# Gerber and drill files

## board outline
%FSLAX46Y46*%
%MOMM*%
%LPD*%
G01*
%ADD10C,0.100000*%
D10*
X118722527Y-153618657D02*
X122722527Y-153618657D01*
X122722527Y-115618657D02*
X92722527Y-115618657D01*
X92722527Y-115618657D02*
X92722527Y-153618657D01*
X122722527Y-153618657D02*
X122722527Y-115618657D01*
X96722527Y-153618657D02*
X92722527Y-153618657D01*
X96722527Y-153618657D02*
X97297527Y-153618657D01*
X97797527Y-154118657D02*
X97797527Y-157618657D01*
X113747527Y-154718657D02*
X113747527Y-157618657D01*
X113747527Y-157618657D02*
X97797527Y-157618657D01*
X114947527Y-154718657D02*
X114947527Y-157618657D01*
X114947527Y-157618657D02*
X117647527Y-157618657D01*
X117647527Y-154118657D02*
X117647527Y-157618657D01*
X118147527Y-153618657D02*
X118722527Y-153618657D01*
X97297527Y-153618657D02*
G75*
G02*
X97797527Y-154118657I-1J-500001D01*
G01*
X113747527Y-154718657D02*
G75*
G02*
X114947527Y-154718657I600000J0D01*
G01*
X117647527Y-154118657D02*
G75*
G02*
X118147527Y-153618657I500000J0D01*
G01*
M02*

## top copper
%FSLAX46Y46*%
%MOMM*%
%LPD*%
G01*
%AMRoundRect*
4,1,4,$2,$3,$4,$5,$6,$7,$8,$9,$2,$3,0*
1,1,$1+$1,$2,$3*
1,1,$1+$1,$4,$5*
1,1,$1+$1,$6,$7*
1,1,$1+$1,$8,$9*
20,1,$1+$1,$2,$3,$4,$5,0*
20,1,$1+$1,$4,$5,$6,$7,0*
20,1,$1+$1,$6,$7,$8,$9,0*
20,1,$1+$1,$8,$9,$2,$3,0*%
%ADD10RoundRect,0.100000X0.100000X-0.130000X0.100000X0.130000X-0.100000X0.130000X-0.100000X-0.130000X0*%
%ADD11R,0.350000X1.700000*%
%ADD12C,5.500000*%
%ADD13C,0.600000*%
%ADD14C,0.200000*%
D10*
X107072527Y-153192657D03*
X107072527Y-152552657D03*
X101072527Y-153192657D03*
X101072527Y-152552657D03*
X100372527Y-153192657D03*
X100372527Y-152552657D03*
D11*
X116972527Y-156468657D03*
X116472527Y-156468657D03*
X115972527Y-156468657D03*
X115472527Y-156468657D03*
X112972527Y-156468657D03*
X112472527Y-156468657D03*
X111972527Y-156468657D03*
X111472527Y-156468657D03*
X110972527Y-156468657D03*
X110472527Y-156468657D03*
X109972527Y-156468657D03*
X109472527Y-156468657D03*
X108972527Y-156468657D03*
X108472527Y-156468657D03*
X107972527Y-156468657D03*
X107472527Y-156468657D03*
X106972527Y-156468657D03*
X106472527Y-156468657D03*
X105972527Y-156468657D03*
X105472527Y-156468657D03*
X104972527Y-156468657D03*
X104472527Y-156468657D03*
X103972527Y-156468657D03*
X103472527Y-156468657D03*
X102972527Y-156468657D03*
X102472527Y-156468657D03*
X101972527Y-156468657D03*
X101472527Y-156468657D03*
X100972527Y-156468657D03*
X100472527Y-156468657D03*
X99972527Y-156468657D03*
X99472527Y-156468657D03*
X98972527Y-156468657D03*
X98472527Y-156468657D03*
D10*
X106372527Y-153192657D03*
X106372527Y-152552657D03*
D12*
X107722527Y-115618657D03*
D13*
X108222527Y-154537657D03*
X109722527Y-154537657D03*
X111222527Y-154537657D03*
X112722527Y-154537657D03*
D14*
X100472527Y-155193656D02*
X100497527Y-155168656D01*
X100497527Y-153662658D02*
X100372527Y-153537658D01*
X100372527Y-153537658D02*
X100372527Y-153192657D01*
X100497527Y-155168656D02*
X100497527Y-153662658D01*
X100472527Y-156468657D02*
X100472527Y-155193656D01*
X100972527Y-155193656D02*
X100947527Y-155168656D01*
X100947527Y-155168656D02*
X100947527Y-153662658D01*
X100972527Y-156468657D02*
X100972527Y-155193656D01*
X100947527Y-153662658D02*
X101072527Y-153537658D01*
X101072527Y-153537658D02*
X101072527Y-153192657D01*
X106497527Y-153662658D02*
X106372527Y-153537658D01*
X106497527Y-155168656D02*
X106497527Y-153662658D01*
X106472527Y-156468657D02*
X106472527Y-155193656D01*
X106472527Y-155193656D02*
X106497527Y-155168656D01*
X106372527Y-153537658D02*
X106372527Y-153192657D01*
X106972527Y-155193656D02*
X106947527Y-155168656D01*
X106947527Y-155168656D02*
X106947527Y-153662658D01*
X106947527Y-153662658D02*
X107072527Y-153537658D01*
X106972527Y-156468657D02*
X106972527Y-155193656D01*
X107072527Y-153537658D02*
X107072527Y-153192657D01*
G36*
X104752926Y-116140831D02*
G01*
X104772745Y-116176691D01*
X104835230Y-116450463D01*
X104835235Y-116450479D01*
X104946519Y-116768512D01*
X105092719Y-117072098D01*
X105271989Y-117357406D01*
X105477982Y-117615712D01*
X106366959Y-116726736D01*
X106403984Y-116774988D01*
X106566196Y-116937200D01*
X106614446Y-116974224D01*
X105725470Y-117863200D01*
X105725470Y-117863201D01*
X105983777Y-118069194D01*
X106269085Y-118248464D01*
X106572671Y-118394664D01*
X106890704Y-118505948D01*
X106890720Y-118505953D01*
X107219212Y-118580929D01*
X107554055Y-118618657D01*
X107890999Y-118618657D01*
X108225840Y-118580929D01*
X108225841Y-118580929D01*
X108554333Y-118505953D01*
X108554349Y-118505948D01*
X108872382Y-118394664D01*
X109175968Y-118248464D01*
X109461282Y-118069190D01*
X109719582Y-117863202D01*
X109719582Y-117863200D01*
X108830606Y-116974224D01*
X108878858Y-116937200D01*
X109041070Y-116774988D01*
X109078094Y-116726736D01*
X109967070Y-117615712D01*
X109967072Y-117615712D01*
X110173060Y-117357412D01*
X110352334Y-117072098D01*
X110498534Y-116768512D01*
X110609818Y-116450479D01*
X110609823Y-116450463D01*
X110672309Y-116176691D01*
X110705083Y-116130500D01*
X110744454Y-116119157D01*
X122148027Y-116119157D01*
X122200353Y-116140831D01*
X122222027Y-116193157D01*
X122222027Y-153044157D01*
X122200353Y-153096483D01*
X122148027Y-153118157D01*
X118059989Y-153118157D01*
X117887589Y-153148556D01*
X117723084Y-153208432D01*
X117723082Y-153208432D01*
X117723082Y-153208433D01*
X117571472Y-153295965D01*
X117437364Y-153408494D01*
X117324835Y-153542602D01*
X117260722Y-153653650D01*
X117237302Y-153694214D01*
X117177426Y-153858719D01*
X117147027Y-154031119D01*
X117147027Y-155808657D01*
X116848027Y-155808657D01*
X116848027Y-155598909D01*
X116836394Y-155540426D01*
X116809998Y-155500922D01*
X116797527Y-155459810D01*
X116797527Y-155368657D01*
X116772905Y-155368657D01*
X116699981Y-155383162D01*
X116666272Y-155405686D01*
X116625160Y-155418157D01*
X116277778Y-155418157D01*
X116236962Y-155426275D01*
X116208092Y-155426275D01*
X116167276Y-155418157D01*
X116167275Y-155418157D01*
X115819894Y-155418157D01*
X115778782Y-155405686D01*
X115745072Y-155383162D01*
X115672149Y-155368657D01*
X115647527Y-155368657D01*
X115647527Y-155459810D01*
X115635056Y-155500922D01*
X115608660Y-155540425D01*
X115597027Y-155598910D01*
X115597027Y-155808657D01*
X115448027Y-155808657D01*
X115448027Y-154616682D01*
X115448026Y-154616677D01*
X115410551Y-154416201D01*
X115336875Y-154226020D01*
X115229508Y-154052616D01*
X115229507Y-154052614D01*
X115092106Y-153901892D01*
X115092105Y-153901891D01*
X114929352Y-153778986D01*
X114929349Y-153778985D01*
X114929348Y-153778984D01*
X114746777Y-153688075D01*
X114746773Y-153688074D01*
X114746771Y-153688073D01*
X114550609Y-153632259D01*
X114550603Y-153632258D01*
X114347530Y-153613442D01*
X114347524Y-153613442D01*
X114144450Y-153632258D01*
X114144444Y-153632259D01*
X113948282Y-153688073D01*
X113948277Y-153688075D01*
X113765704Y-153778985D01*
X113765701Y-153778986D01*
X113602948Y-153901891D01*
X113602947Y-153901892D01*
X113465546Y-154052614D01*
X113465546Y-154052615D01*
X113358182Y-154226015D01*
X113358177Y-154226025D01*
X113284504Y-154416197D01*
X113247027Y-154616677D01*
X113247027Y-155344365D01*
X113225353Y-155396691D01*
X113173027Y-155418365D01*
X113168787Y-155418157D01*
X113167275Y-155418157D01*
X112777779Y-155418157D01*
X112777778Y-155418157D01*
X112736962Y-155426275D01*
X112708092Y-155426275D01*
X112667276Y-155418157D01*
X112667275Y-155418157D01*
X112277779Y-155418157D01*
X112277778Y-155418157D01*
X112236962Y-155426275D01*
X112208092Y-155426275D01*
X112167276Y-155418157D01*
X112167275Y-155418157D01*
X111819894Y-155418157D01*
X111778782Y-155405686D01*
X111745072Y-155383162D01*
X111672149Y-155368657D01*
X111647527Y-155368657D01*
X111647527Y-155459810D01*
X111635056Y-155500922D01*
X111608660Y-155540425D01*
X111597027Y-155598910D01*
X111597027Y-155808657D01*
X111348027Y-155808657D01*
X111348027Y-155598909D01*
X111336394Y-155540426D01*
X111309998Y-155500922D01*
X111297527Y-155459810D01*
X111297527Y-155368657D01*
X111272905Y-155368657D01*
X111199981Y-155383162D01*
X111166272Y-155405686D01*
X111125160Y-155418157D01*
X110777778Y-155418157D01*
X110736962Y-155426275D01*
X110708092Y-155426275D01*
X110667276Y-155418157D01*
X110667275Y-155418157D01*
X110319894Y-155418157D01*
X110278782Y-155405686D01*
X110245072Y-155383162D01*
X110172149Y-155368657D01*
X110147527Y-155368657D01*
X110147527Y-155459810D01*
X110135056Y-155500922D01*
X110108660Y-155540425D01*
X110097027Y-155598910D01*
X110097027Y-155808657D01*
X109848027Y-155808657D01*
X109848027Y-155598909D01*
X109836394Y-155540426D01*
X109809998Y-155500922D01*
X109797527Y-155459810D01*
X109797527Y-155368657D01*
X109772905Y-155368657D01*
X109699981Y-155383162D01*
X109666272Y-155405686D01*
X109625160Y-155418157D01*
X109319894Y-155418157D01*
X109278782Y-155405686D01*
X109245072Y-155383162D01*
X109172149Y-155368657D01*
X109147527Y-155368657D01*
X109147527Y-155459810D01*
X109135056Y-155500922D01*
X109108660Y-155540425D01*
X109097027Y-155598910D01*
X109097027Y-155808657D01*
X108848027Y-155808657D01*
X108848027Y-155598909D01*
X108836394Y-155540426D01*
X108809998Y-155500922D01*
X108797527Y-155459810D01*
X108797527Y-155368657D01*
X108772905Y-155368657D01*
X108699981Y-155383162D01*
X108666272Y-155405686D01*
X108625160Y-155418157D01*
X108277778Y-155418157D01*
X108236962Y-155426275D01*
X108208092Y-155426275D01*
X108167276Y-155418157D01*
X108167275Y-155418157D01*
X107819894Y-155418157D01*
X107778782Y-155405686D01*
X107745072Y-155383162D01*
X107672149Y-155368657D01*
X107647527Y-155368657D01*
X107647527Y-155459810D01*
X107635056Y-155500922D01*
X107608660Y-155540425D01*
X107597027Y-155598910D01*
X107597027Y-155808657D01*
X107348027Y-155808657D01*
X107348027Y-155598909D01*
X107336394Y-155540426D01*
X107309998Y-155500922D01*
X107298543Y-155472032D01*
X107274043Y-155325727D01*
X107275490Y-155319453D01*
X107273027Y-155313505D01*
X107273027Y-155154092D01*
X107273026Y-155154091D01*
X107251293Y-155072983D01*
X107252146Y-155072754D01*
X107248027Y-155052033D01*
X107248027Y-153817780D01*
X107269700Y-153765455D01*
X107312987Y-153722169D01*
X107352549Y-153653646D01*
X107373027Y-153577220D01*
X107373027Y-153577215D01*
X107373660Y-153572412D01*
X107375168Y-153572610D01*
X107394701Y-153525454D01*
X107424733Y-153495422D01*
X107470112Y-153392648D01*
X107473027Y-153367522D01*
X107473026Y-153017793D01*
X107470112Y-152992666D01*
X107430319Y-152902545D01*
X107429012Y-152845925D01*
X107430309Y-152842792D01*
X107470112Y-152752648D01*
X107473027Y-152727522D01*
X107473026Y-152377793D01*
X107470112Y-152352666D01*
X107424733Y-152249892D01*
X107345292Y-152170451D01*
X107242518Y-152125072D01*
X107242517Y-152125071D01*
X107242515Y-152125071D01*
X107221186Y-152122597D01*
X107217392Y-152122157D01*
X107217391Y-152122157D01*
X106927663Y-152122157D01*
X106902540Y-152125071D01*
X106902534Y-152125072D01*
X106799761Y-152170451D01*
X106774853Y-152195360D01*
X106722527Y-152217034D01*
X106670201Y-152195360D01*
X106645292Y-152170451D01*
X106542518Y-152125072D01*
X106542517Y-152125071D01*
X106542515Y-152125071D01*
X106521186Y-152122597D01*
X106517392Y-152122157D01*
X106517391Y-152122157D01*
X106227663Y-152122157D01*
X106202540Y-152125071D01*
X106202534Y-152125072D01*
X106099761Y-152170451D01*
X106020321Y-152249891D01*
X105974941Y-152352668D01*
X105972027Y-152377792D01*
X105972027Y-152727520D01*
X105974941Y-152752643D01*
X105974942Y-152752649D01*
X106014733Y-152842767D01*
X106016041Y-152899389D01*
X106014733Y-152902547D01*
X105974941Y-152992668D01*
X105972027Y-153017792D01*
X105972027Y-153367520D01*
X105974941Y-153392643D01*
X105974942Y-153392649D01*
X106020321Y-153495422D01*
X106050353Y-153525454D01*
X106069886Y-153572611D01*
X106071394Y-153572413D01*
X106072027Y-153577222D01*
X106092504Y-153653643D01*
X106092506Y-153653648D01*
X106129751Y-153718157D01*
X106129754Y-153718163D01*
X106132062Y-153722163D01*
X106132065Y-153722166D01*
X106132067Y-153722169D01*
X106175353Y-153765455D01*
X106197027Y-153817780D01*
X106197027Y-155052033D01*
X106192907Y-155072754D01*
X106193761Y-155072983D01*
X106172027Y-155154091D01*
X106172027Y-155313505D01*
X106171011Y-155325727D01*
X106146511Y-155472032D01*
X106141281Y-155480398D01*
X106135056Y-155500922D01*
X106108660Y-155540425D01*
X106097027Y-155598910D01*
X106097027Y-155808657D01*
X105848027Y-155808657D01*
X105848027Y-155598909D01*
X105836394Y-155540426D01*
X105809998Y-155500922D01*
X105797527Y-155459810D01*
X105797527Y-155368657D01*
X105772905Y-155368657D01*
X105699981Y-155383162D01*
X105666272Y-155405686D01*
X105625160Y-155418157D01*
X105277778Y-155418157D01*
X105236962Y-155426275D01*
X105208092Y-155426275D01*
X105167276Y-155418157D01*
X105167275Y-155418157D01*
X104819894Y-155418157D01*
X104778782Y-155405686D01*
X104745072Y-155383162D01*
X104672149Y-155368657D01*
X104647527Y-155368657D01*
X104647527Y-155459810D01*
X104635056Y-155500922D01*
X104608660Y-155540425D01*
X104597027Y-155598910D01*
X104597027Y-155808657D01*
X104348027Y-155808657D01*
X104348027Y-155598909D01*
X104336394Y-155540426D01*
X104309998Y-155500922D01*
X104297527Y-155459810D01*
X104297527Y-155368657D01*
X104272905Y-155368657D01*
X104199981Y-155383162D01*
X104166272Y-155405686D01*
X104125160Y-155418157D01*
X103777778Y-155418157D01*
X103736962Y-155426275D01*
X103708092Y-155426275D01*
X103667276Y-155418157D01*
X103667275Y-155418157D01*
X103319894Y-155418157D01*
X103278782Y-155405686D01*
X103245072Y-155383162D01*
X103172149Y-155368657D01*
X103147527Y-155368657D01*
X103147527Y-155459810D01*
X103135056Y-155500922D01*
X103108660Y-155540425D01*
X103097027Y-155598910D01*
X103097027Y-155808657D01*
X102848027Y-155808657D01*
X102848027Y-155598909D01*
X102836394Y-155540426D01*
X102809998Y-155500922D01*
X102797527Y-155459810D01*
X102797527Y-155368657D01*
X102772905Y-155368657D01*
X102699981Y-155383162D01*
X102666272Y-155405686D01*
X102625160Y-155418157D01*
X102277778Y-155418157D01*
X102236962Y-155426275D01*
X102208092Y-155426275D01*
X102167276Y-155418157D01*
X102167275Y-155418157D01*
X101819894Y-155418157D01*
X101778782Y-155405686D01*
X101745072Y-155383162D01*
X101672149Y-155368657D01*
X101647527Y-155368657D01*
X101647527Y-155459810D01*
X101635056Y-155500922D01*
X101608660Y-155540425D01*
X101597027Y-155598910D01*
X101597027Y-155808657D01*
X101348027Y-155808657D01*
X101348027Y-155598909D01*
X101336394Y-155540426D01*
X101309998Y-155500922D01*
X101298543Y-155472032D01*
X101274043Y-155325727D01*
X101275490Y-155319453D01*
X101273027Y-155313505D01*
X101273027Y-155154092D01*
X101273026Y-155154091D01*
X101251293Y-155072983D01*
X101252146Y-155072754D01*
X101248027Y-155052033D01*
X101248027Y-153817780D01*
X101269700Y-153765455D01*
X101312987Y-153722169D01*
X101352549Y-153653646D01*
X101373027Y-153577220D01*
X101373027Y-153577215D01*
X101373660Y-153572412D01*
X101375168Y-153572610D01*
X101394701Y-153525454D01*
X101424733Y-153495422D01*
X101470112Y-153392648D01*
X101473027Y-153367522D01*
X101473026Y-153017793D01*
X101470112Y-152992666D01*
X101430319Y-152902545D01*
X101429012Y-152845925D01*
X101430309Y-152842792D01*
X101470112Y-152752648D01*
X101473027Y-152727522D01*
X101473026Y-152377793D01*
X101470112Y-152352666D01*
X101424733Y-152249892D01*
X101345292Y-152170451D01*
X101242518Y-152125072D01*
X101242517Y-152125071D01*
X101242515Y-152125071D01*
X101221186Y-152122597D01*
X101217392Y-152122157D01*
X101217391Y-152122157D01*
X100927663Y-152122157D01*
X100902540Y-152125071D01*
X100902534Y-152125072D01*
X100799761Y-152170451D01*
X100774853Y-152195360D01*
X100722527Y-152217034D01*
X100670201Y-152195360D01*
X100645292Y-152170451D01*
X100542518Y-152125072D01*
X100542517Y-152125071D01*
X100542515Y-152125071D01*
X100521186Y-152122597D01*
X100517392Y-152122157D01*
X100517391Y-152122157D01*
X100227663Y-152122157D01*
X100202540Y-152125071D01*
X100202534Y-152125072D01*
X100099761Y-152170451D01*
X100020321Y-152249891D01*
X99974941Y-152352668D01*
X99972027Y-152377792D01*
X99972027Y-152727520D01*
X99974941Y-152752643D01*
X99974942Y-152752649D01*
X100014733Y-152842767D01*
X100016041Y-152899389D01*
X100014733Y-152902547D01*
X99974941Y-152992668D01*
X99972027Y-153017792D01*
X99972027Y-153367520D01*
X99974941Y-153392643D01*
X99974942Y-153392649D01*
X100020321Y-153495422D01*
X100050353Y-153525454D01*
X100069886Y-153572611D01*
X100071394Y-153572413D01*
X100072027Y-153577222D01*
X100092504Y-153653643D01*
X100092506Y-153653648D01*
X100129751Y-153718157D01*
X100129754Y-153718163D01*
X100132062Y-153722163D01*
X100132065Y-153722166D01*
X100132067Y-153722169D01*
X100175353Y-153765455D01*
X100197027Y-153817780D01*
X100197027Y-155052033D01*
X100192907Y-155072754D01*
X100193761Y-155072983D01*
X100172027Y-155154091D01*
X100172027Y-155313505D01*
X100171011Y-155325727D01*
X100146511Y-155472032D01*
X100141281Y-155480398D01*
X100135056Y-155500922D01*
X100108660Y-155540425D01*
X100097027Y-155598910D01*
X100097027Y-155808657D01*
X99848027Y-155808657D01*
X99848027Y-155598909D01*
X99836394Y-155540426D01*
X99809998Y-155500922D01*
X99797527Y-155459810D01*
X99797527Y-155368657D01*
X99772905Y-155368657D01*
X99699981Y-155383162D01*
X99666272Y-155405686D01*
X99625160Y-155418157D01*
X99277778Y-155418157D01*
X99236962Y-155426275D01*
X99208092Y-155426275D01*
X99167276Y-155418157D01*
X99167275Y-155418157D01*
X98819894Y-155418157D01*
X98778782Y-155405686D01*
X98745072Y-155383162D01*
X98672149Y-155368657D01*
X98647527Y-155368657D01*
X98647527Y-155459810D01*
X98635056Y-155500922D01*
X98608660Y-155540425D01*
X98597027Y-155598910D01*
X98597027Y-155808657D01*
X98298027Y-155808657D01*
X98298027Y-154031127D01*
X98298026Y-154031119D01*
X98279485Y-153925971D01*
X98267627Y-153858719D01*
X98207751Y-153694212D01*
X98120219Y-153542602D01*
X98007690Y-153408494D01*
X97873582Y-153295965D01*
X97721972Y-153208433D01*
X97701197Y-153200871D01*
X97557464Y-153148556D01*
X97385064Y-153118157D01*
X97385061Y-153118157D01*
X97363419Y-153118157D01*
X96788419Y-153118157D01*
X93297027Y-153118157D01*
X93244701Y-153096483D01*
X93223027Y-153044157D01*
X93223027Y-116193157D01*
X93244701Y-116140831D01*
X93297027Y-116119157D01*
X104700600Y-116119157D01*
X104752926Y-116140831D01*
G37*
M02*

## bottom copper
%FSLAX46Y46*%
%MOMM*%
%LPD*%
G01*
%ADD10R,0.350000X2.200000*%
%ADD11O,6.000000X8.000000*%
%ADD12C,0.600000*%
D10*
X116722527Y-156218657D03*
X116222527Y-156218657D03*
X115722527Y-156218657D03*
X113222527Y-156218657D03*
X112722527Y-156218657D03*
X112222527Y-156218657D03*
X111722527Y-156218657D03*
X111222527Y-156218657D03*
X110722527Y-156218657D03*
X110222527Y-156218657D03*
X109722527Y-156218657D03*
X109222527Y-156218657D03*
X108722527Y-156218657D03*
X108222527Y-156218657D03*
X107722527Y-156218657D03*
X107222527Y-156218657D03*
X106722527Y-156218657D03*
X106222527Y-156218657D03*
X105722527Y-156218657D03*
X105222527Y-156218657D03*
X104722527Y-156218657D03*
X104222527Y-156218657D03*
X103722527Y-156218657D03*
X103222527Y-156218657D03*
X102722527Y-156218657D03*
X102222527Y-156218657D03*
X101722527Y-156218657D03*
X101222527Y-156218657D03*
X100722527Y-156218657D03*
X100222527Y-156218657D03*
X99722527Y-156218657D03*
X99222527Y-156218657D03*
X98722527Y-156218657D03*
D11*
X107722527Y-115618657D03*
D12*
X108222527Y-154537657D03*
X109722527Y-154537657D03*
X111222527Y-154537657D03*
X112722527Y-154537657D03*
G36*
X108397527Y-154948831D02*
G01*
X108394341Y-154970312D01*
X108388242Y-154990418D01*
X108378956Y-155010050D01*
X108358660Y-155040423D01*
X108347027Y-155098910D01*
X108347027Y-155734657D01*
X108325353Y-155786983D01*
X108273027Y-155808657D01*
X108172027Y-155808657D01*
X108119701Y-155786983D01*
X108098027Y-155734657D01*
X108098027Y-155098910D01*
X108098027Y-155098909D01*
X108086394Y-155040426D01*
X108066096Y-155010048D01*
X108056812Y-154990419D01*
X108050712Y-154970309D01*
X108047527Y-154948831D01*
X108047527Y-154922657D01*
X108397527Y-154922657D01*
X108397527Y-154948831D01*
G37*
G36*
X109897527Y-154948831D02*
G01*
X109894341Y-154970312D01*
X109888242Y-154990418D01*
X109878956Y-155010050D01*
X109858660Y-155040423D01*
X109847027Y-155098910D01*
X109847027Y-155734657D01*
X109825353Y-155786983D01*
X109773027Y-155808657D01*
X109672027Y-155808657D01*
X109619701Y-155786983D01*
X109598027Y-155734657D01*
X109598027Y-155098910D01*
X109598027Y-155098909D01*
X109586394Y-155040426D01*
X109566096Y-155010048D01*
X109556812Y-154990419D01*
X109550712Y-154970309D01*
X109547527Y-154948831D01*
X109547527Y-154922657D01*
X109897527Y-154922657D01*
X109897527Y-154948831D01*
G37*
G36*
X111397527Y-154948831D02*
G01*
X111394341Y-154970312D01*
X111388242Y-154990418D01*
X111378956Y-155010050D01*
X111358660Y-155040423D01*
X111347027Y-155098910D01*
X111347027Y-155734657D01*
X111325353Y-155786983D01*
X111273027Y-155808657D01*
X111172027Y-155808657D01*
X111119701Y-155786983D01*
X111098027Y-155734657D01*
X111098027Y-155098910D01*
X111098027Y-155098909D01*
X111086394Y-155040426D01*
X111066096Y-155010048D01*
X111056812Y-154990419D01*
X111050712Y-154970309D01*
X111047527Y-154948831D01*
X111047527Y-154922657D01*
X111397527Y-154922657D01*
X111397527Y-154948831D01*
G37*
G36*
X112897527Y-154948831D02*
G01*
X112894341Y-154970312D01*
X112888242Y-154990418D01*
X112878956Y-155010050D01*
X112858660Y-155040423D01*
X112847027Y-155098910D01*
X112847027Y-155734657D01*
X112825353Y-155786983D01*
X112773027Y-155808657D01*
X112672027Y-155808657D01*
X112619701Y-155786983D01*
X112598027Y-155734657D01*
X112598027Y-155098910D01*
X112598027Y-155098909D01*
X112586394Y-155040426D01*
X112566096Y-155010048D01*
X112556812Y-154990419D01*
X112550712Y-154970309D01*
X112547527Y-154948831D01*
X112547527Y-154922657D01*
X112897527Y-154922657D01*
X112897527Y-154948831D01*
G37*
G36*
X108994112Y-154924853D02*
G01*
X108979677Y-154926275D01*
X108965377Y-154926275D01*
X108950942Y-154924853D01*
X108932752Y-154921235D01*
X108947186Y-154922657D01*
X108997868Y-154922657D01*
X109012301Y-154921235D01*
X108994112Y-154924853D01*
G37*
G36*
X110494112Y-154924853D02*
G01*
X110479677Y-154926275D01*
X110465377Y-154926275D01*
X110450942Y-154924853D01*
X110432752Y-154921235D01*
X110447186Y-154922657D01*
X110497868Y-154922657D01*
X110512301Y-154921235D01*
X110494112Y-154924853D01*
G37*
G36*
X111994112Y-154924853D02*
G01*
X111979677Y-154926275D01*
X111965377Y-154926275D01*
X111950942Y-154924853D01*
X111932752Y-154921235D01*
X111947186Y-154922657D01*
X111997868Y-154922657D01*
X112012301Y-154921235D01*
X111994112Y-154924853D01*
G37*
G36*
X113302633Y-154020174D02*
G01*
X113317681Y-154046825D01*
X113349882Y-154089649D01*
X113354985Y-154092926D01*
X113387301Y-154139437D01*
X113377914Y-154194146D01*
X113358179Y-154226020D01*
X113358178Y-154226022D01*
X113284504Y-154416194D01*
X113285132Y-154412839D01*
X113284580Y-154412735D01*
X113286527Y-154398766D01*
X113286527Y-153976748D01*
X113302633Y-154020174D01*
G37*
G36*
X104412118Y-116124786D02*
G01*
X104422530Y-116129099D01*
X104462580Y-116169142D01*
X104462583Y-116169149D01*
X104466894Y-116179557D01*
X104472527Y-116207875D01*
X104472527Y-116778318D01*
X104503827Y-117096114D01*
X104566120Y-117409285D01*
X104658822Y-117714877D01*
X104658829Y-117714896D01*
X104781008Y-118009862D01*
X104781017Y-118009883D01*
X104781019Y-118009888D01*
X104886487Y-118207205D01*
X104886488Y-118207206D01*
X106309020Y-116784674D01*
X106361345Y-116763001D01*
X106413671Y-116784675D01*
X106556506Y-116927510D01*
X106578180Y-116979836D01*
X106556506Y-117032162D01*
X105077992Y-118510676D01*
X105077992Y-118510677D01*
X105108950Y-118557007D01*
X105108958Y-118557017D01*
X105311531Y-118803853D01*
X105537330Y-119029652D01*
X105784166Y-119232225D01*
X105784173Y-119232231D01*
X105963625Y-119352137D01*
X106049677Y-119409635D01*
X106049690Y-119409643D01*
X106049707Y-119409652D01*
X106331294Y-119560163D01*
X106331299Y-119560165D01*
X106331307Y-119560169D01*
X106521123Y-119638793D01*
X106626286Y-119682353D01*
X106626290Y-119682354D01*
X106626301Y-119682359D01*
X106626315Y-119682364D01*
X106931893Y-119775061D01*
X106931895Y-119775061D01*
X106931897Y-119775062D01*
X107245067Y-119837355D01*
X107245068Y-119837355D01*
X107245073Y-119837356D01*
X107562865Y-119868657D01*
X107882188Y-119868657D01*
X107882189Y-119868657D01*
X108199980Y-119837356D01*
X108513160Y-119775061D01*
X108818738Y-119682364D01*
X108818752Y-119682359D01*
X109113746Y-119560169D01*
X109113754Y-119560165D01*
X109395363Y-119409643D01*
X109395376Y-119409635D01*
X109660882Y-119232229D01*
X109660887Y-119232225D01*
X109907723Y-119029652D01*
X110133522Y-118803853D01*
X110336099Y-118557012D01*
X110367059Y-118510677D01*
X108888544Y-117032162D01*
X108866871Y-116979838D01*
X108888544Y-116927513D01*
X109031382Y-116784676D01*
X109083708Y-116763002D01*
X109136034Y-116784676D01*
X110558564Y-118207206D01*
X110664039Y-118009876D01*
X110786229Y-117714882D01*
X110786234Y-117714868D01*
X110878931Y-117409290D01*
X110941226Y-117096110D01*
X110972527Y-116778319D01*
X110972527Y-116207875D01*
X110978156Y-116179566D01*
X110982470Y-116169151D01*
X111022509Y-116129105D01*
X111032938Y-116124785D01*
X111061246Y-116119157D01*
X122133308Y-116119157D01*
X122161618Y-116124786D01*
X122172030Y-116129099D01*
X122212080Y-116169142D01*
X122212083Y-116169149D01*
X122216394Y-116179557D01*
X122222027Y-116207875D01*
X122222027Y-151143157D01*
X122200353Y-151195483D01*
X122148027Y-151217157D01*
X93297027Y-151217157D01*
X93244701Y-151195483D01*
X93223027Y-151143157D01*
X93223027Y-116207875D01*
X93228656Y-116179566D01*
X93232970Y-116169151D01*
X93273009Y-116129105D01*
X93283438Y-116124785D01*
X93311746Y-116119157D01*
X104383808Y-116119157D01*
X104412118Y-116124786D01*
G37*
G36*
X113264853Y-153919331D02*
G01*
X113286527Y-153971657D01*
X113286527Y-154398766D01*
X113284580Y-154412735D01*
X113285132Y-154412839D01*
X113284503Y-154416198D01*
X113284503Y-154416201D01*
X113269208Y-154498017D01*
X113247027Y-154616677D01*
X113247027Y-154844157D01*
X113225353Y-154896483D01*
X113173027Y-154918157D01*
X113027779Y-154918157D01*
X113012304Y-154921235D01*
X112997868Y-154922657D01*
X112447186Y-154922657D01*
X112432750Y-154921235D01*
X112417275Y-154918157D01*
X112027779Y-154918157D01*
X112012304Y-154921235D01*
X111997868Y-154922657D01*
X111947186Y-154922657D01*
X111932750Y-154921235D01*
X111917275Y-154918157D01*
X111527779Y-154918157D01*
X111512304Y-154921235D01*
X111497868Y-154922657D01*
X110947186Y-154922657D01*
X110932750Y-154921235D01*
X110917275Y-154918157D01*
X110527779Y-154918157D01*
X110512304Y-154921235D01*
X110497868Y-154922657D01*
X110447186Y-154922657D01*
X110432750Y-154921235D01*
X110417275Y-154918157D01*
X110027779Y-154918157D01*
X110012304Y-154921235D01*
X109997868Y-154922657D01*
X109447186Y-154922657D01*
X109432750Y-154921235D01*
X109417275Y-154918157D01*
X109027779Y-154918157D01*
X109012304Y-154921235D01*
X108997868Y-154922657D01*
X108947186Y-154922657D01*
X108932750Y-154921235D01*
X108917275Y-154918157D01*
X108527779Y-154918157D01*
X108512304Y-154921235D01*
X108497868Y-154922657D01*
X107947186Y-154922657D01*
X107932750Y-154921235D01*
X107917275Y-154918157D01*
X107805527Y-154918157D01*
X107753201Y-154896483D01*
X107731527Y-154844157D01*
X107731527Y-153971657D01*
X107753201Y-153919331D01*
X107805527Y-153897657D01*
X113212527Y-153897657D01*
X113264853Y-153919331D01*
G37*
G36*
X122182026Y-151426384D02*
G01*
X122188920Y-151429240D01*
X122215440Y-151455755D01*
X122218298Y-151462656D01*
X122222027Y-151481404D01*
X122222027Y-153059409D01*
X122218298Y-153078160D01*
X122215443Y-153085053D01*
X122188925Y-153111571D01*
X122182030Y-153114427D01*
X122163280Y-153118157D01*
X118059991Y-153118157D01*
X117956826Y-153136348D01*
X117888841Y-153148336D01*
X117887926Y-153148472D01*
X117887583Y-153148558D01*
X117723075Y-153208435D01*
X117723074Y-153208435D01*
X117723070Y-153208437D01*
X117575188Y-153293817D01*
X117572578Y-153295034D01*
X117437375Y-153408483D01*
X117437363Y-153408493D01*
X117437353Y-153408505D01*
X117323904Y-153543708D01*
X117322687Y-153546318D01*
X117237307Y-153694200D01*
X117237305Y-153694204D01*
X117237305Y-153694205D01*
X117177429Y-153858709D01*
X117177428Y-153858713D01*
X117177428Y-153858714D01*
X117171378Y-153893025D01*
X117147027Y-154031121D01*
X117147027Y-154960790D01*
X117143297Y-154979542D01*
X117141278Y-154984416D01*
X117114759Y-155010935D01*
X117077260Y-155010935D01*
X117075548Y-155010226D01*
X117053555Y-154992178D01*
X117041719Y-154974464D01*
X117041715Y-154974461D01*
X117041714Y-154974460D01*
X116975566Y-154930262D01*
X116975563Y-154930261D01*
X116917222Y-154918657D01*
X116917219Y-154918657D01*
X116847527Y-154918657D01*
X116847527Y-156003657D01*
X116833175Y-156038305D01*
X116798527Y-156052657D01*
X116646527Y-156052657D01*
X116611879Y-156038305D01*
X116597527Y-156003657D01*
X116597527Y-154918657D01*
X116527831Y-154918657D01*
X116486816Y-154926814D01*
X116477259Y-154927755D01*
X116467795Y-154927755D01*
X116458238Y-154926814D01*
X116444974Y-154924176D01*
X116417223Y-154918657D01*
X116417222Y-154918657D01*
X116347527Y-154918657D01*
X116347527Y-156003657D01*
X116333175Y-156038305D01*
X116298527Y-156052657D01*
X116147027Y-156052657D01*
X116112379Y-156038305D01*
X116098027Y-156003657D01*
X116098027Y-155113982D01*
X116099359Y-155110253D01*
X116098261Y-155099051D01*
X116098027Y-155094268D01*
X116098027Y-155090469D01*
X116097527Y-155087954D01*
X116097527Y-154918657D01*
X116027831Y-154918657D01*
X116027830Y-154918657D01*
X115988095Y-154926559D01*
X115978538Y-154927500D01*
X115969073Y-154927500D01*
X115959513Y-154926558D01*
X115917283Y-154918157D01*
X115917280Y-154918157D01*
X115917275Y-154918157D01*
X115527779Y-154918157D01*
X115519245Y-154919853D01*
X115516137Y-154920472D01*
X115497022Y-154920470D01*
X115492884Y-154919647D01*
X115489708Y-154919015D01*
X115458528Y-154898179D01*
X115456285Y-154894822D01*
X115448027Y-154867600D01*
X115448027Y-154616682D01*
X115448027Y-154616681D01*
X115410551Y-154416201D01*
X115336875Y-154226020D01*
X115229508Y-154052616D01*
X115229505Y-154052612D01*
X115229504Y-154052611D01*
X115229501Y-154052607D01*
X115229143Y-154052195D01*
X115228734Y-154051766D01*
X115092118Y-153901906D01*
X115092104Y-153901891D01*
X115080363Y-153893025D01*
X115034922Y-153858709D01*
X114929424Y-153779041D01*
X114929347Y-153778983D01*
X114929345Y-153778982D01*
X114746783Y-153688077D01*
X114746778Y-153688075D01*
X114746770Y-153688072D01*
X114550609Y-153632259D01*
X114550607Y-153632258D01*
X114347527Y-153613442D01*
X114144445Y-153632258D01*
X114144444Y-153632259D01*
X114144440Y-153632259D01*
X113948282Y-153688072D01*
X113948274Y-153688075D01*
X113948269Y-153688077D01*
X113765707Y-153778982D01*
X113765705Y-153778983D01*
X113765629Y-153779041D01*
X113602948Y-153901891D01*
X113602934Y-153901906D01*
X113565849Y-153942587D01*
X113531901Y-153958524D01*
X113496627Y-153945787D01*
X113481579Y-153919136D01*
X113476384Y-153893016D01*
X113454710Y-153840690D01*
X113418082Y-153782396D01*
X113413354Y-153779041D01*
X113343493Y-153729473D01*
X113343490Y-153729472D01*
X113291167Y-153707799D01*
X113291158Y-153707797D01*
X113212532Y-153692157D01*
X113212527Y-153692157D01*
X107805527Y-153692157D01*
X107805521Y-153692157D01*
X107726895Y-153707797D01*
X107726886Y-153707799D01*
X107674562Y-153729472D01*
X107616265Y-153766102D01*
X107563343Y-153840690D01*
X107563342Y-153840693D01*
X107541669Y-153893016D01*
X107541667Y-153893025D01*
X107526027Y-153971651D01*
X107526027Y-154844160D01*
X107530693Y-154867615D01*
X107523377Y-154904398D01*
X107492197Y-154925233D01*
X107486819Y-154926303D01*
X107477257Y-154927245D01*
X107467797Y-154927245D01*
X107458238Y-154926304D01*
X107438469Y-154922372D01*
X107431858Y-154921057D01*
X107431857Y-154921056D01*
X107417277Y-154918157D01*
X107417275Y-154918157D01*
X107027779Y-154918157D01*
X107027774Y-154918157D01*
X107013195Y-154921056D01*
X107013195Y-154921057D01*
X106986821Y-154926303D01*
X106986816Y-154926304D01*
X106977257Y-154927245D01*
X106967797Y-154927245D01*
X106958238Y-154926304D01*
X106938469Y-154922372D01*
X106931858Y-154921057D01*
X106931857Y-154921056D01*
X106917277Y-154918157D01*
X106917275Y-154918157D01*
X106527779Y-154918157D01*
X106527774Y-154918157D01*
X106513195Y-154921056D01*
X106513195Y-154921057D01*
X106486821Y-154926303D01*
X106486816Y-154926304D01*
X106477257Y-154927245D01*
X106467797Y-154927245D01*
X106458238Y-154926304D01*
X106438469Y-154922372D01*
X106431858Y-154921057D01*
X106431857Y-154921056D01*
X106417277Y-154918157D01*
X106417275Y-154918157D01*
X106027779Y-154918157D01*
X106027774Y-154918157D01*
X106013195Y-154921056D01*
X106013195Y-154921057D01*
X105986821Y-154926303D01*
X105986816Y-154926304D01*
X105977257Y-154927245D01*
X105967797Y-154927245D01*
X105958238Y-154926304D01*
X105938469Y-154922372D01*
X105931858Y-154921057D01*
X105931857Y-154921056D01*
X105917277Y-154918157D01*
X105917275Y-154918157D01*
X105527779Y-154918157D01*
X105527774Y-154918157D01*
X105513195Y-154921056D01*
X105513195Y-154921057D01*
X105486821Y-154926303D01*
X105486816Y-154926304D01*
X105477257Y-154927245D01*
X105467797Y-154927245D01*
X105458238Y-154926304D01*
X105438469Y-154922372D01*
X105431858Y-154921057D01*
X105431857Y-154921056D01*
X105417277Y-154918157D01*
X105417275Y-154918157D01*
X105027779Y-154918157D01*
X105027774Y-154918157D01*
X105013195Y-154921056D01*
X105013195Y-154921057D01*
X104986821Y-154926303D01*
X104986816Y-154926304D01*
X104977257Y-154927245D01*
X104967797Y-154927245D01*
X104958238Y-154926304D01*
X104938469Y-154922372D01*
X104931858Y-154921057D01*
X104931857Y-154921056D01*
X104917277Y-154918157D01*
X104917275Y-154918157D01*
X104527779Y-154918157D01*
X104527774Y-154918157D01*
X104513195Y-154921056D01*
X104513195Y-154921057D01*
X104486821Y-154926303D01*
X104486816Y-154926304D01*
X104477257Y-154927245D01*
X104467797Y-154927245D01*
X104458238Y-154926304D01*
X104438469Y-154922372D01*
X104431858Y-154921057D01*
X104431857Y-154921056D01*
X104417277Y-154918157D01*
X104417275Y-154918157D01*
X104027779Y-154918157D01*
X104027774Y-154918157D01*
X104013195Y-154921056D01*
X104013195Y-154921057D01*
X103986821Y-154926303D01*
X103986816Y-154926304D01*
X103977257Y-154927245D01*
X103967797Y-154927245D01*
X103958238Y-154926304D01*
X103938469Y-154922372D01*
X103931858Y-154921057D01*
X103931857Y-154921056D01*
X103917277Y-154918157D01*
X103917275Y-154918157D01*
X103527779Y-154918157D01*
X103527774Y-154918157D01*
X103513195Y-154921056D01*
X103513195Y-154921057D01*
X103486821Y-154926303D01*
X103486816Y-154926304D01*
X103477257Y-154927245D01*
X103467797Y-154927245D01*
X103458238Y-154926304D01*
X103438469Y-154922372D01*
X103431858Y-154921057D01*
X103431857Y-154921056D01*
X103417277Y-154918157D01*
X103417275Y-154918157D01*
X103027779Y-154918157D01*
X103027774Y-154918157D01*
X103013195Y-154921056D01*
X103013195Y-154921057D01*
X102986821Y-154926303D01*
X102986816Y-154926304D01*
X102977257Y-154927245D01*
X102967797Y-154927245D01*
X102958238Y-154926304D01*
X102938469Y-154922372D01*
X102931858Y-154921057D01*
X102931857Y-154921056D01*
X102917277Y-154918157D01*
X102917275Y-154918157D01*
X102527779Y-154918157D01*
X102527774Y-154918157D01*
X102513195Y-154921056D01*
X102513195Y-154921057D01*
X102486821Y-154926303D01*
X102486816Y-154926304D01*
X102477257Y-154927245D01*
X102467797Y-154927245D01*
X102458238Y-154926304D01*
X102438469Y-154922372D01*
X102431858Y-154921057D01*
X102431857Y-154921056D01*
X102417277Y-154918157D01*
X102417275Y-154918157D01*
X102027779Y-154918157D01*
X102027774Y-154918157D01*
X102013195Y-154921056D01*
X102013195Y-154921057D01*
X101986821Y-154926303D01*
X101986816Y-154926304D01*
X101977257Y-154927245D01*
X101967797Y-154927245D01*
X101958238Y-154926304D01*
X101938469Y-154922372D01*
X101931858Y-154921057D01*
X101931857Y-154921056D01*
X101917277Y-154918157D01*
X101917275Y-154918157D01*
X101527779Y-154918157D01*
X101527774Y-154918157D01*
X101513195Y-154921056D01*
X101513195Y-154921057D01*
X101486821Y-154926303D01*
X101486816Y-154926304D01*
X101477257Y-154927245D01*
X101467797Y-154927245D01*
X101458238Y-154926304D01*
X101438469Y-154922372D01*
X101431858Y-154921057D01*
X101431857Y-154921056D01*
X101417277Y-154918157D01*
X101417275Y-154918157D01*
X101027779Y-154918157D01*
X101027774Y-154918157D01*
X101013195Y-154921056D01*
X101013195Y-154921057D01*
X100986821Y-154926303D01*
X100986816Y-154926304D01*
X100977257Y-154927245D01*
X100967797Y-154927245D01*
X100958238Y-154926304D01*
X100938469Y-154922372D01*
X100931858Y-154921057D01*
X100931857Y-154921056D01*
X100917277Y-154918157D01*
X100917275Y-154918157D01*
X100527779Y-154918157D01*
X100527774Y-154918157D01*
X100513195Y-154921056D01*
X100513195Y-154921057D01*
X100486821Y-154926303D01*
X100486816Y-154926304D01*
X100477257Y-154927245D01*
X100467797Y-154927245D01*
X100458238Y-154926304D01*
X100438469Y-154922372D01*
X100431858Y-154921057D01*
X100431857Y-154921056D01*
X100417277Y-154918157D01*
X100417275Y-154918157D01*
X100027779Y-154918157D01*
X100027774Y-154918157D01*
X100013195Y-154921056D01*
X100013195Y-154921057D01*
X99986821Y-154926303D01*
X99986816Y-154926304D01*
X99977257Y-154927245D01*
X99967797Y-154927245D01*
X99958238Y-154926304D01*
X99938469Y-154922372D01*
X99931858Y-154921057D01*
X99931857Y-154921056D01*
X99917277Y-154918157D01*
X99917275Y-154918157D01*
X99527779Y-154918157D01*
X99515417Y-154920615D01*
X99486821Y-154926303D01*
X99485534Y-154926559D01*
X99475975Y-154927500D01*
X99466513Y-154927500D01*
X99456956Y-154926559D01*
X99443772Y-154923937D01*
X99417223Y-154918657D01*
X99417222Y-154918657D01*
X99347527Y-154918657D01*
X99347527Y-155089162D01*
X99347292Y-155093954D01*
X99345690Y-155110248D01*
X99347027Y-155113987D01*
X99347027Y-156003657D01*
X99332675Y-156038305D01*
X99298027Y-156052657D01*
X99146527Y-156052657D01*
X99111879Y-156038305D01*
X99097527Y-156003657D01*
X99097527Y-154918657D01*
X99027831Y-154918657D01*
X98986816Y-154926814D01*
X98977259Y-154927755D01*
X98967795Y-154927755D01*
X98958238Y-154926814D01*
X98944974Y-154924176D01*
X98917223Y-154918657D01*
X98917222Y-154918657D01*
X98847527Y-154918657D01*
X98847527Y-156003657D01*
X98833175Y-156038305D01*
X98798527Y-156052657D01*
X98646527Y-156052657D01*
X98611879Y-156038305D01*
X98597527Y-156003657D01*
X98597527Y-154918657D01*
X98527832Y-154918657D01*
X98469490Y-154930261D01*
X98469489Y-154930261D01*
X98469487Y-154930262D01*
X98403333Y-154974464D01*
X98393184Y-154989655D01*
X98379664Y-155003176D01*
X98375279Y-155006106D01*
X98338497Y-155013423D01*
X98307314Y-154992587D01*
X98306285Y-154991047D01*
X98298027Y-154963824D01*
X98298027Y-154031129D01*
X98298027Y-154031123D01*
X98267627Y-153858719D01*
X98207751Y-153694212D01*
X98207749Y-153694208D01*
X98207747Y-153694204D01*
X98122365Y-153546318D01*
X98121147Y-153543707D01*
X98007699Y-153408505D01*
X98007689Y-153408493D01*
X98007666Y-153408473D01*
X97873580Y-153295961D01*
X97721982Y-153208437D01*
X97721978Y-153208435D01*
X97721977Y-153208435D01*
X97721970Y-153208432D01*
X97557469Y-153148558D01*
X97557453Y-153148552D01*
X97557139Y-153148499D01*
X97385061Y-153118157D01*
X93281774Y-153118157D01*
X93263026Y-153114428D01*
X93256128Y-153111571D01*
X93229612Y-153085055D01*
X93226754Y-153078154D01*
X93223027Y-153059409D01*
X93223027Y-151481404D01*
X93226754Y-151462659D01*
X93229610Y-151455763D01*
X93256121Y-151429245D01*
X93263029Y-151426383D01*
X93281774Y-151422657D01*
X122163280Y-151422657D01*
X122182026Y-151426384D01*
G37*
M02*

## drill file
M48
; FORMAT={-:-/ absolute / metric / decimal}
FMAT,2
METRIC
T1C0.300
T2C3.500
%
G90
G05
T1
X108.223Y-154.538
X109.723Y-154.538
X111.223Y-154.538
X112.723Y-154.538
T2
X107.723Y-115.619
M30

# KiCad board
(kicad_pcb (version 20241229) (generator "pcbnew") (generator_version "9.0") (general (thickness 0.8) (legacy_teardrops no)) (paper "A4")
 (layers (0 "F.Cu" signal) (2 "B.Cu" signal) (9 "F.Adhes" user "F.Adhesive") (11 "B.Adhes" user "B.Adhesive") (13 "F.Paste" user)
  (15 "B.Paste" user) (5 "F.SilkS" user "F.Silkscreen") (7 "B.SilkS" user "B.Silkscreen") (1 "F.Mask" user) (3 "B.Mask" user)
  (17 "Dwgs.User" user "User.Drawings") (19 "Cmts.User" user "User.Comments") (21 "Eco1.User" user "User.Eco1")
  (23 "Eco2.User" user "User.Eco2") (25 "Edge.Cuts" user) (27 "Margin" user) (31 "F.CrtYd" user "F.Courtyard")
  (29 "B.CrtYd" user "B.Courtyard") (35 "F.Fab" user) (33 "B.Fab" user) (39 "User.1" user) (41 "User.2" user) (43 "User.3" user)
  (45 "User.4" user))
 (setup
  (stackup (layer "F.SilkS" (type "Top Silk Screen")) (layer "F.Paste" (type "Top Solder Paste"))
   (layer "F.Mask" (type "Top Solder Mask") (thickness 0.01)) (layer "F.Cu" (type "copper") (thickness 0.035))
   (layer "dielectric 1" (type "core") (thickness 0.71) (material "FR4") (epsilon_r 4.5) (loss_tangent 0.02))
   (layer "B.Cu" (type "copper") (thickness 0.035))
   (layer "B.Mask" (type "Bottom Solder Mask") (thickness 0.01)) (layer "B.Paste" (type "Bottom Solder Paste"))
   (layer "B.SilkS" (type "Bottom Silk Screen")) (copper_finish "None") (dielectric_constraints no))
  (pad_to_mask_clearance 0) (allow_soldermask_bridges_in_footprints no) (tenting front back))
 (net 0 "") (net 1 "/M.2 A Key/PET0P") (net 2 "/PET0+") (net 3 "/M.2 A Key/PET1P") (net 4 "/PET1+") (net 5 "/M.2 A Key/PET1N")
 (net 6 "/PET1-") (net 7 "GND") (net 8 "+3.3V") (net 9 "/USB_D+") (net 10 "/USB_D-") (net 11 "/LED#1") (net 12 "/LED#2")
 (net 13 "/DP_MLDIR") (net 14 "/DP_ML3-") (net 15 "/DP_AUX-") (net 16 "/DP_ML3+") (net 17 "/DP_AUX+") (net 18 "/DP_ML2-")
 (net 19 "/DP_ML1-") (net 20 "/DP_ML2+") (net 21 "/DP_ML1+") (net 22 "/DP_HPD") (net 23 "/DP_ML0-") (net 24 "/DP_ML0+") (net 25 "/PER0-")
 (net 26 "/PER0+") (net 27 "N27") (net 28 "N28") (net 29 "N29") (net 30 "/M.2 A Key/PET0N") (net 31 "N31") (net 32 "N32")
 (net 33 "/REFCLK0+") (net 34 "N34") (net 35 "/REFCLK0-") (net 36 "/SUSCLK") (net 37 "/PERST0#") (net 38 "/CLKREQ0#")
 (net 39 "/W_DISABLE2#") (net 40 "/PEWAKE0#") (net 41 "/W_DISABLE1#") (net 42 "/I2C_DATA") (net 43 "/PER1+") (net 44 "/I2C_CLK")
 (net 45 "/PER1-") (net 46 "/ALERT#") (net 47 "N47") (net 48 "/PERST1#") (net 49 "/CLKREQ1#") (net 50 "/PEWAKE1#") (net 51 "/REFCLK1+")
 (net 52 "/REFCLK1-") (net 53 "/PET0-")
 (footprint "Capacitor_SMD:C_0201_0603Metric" (layer "F.Cu") (at 107.072527 152.872657 90)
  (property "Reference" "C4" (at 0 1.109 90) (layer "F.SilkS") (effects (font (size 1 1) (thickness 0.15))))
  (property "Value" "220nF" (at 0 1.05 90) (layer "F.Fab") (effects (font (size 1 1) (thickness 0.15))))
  (pad "" smd roundrect (at -0.345 0 90) (size 0.318 0.36) (layers "F.Paste") (roundrect_rratio 0.25))
  (pad "" smd roundrect (at 0.345 0 90) (size 0.318 0.36) (layers "F.Paste") (roundrect_rratio 0.25))
  (pad "1" smd roundrect (at -0.32 0 90) (size 0.46 0.4) (layers "F.Cu" "F.Mask") (roundrect_rratio 0.25) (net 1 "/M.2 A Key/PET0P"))
  (pad "2" smd roundrect (at 0.32 0 90) (size 0.46 0.4) (layers "F.Cu" "F.Mask") (roundrect_rratio 0.25) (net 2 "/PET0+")))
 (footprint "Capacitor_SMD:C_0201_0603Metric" (layer "F.Cu") (at 101.072527 152.872657 90)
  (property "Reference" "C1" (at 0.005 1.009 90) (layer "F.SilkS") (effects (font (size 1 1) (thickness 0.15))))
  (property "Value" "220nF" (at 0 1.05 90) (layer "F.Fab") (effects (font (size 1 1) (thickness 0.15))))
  (pad "" smd roundrect (at -0.345 0 90) (size 0.318 0.36) (layers "F.Paste") (roundrect_rratio 0.25))
  (pad "" smd roundrect (at 0.345 0 90) (size 0.318 0.36) (layers "F.Paste") (roundrect_rratio 0.25))
  (pad "1" smd roundrect (at -0.32 0 90) (size 0.46 0.4) (layers "F.Cu" "F.Mask") (roundrect_rratio 0.25) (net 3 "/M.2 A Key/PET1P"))
  (pad "2" smd roundrect (at 0.32 0 90) (size 0.46 0.4) (layers "F.Cu" "F.Mask") (roundrect_rratio 0.25) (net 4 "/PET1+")))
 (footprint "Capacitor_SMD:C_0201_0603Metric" (layer "F.Cu") (at 100.372527 152.872657 90)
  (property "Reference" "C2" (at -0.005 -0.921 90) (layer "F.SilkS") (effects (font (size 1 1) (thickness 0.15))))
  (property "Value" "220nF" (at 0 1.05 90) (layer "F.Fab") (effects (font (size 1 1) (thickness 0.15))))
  (pad "" smd roundrect (at -0.345 0 90) (size 0.318 0.36) (layers "F.Paste") (roundrect_rratio 0.25))
  (pad "" smd roundrect (at 0.345 0 90) (size 0.318 0.36) (layers "F.Paste") (roundrect_rratio 0.25))
  (pad "1" smd roundrect (at -0.32 0 90) (size 0.46 0.4) (layers "F.Cu" "F.Mask") (roundrect_rratio 0.25) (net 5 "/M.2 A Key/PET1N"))
  (pad "2" smd roundrect (at 0.32 0 90) (size 0.46 0.4) (layers "F.Cu" "F.Mask") (roundrect_rratio 0.25) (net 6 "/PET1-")))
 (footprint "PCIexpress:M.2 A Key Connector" (layer "F.Cu") (at 107.722527 156.508657)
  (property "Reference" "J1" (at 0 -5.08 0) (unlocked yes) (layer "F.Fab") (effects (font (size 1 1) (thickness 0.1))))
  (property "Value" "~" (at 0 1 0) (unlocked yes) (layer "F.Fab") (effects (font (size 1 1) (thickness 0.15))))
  (fp_line (start -11 -2.89) (end -10.425 -2.89) (stroke (width 0.1) (type default)) (layer "Edge.Cuts"))
  (fp_line (start -9.925 -2.39) (end -9.925 1.11) (stroke (width 0.1) (type default)) (layer "Edge.Cuts"))
  (fp_line (start 6.025 -1.79) (end 6.025 1.11) (stroke (width 0.1) (type default)) (layer "Edge.Cuts"))
  (fp_line (start 6.025 1.11) (end -9.925 1.11) (stroke (width 0.1) (type default)) (layer "Edge.Cuts"))
  (fp_line (start 7.225 -1.79) (end 7.225 1.11) (stroke (width 0.1) (type default)) (layer "Edge.Cuts"))
  (fp_line (start 7.225 1.11) (end 9.925 1.11) (stroke (width 0.1) (type default)) (layer "Edge.Cuts"))
  (fp_line (start 9.925 -2.39) (end 9.925 1.11) (stroke (width 0.1) (type default)) (layer "Edge.Cuts"))
  (fp_line (start 10.425 -2.89) (end 11 -2.89) (stroke (width 0.1) (type default)) (layer "Edge.Cuts"))
  (fp_arc (start -10.425 -2.89) (mid -10.071447 -2.743553) (end -9.925 -2.39) (stroke (width 0.1) (type default)) (layer "Edge.Cuts"))
  (fp_arc (start 6.025 -1.79) (mid 6.625 -2.39) (end 7.225 -1.79) (stroke (width 0.1) (type default)) (layer "Edge.Cuts"))
  (fp_arc (start 9.925 -2.39) (mid 10.071447 -2.743553) (end 10.425 -2.89) (stroke (width 0.1) (type default)) (layer "Edge.Cuts"))
  (pad "1" smd rect (at 9.25 -0.04 180) (size 0.35 1.7) (layers "F.Cu") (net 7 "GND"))
  (pad "2" smd rect (at 9 -0.29 180) (size 0.35 2.2) (layers "B.Cu") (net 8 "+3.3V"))
  (pad "3" smd rect (at 8.75 -0.04 180) (size 0.35 1.7) (layers "F.Cu") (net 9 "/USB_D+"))
  (pad "4" smd rect (at 8.5 -0.29 180) (size 0.35 2.2) (layers "B.Cu") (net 8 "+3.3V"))
  (pad "5" smd rect (at 8.25 -0.04 180) (size 0.35 1.7) (layers "F.Cu") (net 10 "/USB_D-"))
  (pad "6" smd rect (at 8 -0.29 180) (size 0.35 2.2) (layers "B.Cu") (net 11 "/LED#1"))
  (pad "7" smd rect (at 7.75 -0.04 180) (size 0.35 1.7) (layers "F.Cu") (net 7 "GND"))
  (pad "16" smd rect (at 5.5 -0.29 180) (size 0.35 2.2) (layers "B.Cu") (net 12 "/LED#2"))
  (pad "17" smd rect (at 5.25 -0.04 180) (size 0.35 1.7) (layers "F.Cu") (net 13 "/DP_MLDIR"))
  (pad "18" smd rect (at 5 -0.29 180) (size 0.35 2.2) (layers "B.Cu") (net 7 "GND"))
  (pad "19" smd rect (at 4.75 -0.04 180) (size 0.35 1.7) (layers "F.Cu") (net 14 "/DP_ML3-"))
  (pad "20" smd rect (at 4.5 -0.29 180) (size 0.35 2.2) (layers "B.Cu") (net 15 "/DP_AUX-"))
  (pad "21" smd rect (at 4.25 -0.04 180) (size 0.35 1.7) (layers "F.Cu") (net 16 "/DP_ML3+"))
  (pad "22" smd rect (at 4 -0.29 180) (size 0.35 2.2) (layers "B.Cu") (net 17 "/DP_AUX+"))
  (pad "23" smd rect (at 3.75 -0.04 180) (size 0.35 1.7) (layers "F.Cu") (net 7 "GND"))
  (pad "24" smd rect (at 3.5 -0.29 180) (size 0.35 2.2) (layers "B.Cu") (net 7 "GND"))
  (pad "25" smd rect (at 3.25 -0.04 180) (size 0.35 1.7) (layers "F.Cu") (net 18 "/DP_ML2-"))
  (pad "26" smd rect (at 3 -0.29 180) (size 0.35 2.2) (layers "B.Cu") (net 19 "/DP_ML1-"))
  (pad "27" smd rect (at 2.75 -0.04 180) (size 0.35 1.7) (layers "F.Cu") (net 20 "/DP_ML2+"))
  (pad "28" smd rect (at 2.5 -0.29 180) (size 0.35 2.2) (layers "B.Cu") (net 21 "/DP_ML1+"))
  (pad "29" smd rect (at 2.25 -0.04 180) (size 0.35 1.7) (layers "F.Cu") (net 7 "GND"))
  (pad "30" smd rect (at 2 -0.29 180) (size 0.35 2.2) (layers "B.Cu") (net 7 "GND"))
  (pad "31" smd rect (at 1.75 -0.04 180) (size 0.35 1.7) (layers "F.Cu") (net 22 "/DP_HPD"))
  (pad "32" smd rect (at 1.5 -0.29 180) (size 0.35 2.2) (layers "B.Cu") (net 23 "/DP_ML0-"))
  (pad "33" smd rect (at 1.25 -0.04 180) (size 0.35 1.7) (layers "F.Cu") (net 7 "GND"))
  (pad "34" smd rect (at 1 -0.29 180) (size 0.35 2.2) (layers "B.Cu") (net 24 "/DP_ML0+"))
  (pad "35" smd rect (at 0.75 -0.04 180) (size 0.35 1.7) (layers "F.Cu") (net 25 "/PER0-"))
  (pad "36" smd rect (at 0.5 -0.29 180) (size 0.35 2.2) (layers "B.Cu") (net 7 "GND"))
  (pad "37" smd rect (at 0.25 -0.04 180) (size 0.35 1.7) (layers "F.Cu") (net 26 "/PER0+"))
  (pad "38" smd rect (at 0 -0.29 180) (size 0.35 2.2) (layers "B.Cu") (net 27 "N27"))
  (pad "39" smd rect (at -0.25 -0.04 180) (size 0.35 1.7) (layers "F.Cu") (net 7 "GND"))
  (pad "40" smd rect (at -0.5 -0.29 180) (size 0.35 2.2) (layers "B.Cu") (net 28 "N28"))
  (pad "41" smd rect (at -0.75 -0.04 180) (size 0.35 1.7) (layers "F.Cu") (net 1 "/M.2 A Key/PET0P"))
  (pad "42" smd rect (at -1 -0.29 180) (size 0.35 2.2) (layers "B.Cu") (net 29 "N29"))
  (pad "43" smd rect (at -1.25 -0.04 180) (size 0.35 1.7) (layers "F.Cu") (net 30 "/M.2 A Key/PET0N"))
  (pad "44" smd rect (at -1.5 -0.29 180) (size 0.35 2.2) (layers "B.Cu") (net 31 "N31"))
  (pad "45" smd rect (at -1.75 -0.04 180) (size 0.35 1.7) (layers "F.Cu") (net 7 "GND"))
  (pad "46" smd rect (at -2 -0.29 180) (size 0.35 2.2) (layers "B.Cu") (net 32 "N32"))
  (pad "47" smd rect (at -2.25 -0.04 180) (size 0.35 1.7) (layers "F.Cu") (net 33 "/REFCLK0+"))
  (pad "48" smd rect (at -2.5 -0.29 180) (size 0.35 2.2) (layers "B.Cu") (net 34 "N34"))
  (pad "49" smd rect (at -2.75 -0.04 180) (size 0.35 1.7) (layers "F.Cu") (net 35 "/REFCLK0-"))
  (pad "50" smd rect (at -3 -0.29 180) (size 0.35 2.2) (layers "B.Cu") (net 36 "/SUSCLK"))
  (pad "51" smd rect (at -3.25 -0.04 180) (size 0.35 1.7) (layers "F.Cu") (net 7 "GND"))
  (pad "52" smd rect (at -3.5 -0.29 180) (size 0.35 2.2) (layers "B.Cu") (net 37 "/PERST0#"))
  (pad "53" smd rect (at -3.75 -0.04 180) (size 0.35 1.7) (layers "F.Cu") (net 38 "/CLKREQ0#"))
  (pad "54" smd rect (at -4 -0.29 180) (size 0.35 2.2) (layers "B.Cu") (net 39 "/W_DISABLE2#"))
  (pad "55" smd rect (at -4.25 -0.04 180) (size 0.35 1.7) (layers "F.Cu") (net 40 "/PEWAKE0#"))
  (pad "56" smd rect (at -4.5 -0.29 180) (size 0.35 2.2) (layers "B.Cu") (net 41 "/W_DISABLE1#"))
  (pad "57" smd rect (at -4.75 -0.04 180) (size 0.35 1.7) (layers "F.Cu") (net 7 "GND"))
  (pad "58" smd rect (at -5 -0.29 180) (size 0.35 2.2) (layers "B.Cu") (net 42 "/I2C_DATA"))
  (pad "59" smd rect (at -5.25 -0.04 180) (size 0.35 1.7) (layers "F.Cu") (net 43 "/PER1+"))
  (pad "60" smd rect (at -5.5 -0.29 180) (size 0.35 2.2) (layers "B.Cu") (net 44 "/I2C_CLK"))
  (pad "61" smd rect (at -5.75 -0.04 180) (size 0.35 1.7) (layers "F.Cu") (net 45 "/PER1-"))
  (pad "62" smd rect (at -6 -0.29 180) (size 0.35 2.2) (layers "B.Cu") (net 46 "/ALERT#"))
  (pad "63" smd rect (at -6.25 -0.04 180) (size 0.35 1.7) (layers "F.Cu") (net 7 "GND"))
  (pad "64" smd rect (at -6.5 -0.29 180) (size 0.35 2.2) (layers "B.Cu") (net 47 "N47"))
  (pad "65" smd rect (at -6.75 -0.04 180) (size 0.35 1.7) (layers "F.Cu") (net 3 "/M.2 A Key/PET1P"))
  (pad "66" smd rect (at -7 -0.29 180) (size 0.35 2.2) (layers "B.Cu") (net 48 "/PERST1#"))
  (pad "67" smd rect (at -7.25 -0.04 180) (size 0.35 1.7) (layers "F.Cu") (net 5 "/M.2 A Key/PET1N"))
  (pad "68" smd rect (at -7.5 -0.29 180) (size 0.35 2.2) (layers "B.Cu") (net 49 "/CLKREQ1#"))
  (pad "69" smd rect (at -7.75 -0.04 180) (size 0.35 1.7) (layers "F.Cu") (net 7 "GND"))
  (pad "70" smd rect (at -8 -0.29 180) (size 0.35 2.2) (layers "B.Cu") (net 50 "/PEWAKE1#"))
  (pad "71" smd rect (at -8.25 -0.04 180) (size 0.35 1.7) (layers "F.Cu") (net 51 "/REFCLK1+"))
  (pad "72" smd rect (at -8.5 -0.29 180) (size 0.35 2.2) (layers "B.Cu") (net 8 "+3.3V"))
  (pad "73" smd rect (at -8.75 -0.04 180) (size 0.35 1.7) (layers "F.Cu") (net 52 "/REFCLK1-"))
  (pad "74" smd rect (at -9 -0.29 180) (size 0.35 2.2) (layers "B.Cu") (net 8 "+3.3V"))
  (pad "75" smd rect (at -9.25 -0.04 180) (size 0.35 1.7) (layers "F.Cu") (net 7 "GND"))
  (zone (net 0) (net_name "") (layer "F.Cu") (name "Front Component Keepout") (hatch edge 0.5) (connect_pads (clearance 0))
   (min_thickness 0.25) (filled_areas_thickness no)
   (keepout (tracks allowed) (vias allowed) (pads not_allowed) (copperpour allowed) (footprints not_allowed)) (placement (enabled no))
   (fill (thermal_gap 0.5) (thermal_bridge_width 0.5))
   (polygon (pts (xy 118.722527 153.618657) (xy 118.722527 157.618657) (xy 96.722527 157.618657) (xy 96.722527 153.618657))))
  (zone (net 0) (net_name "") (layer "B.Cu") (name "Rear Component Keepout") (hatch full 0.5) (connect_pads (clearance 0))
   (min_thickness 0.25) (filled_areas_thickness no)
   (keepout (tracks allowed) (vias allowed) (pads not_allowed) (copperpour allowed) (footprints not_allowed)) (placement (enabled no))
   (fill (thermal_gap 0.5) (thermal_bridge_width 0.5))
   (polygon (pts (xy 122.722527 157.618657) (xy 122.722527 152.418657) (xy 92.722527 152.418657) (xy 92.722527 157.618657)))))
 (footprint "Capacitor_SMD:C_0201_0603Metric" (layer "F.Cu") (at 106.372527 152.872657 90)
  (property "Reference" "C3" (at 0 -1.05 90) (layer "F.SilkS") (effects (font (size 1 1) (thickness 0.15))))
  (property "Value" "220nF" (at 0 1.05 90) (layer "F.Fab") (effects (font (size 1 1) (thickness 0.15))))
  (pad "" smd roundrect (at -0.345 0 90) (size 0.318 0.36) (layers "F.Paste") (roundrect_rratio 0.25))
  (pad "" smd roundrect (at 0.345 0 90) (size 0.318 0.36) (layers "F.Paste") (roundrect_rratio 0.25))
  (pad "1" smd roundrect (at -0.32 0 90) (size 0.46 0.4) (layers "F.Cu" "F.Mask") (roundrect_rratio 0.25) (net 30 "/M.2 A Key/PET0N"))
  (pad "2" smd roundrect (at 0.32 0 90) (size 0.46 0.4) (layers "F.Cu" "F.Mask") (roundrect_rratio 0.25) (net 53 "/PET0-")))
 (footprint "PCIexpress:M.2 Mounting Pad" (layer "F.Cu") (at 107.722527 115.618657)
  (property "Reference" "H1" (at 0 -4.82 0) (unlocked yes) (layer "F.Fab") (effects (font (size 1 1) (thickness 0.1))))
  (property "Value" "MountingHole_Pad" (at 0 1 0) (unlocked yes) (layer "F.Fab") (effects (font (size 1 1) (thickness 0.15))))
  (pad "1" thru_hole circle (at 0 0) (size 5.5 5.5) (drill 3.5) (layers "*.Cu" "*.Mask") (remove_unused_layers no) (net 7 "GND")
   (padstack (mode front_inner_back)
    (layer "Inner" (shape circle) (size 5.5 5.5) (zone_connect -1))
    (layer "B.Cu" (shape oval) (size 6 8) (thermal_bridge_angle 45) (zone_connect -1)))))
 (gr_line (start 118.722527 153.618657) (end 122.722527 153.618657) (stroke (width 0.1) (type default)) (layer "Edge.Cuts"))
 (gr_line (start 122.722527 115.618657) (end 92.722527 115.618657) (stroke (width 0.1) (type solid)) (layer "Edge.Cuts"))
 (gr_line (start 92.722527 115.618657) (end 92.722527 153.618657) (stroke (width 0.1) (type default)) (layer "Edge.Cuts"))
 (gr_line (start 122.722527 153.618657) (end 122.722527 115.618657) (stroke (width 0.1) (type default)) (layer "Edge.Cuts"))
 (gr_line (start 96.722527 153.618657) (end 92.722527 153.618657) (stroke (width 0.1) (type default)) (layer "Edge.Cuts"))
 (via (at 108.222527 154.537657) (size 0.6) (drill 0.3) (layers "F.Cu" "B.Cu") (free yes) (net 7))
 (via (at 109.722527 154.537657) (size 0.6) (drill 0.3) (layers "F.Cu" "B.Cu") (free yes) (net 7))
 (via (at 111.222527 154.537657) (size 0.6) (drill 0.3) (layers "F.Cu" "B.Cu") (free yes) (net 7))
 (via (at 112.722527 154.537657) (size 0.6) (drill 0.3) (layers "F.Cu" "B.Cu") (free yes) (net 7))
 (segment (start 100.472527 155.193656) (end 100.497527 155.168656) (width 0.2) (layer "F.Cu") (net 5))
 (segment (start 100.497527 153.662658) (end 100.372527 153.537658) (width 0.2) (layer "F.Cu") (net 5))
 (segment (start 100.372527 153.537658) (end 100.372527 153.192657) (width 0.2) (layer "F.Cu") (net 5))
 (segment (start 100.497527 155.168656) (end 100.497527 153.662658) (width 0.2) (layer "F.Cu") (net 5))
 (segment (start 100.472527 156.468657) (end 100.472527 155.193656) (width 0.2) (layer "F.Cu") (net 5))
 (segment (start 100.972527 155.193656) (end 100.947527 155.168656) (width 0.2) (layer "F.Cu") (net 3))
 (segment (start 100.947527 155.168656) (end 100.947527 153.662658) (width 0.2) (layer "F.Cu") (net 3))
 (segment (start 100.972527 156.468657) (end 100.972527 155.193656) (width 0.2) (layer "F.Cu") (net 3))
 (segment (start 100.947527 153.662658) (end 101.072527 153.537658) (width 0.2) (layer "F.Cu") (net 3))
 (segment (start 101.072527 153.537658) (end 101.072527 153.192657) (width 0.2) (layer "F.Cu") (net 3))
 (segment (start 106.497527 153.662658) (end 106.372527 153.537658) (width 0.2) (layer "F.Cu") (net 30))
 (segment (start 106.497527 155.168656) (end 106.497527 153.662658) (width 0.2) (layer "F.Cu") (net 30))
 (segment (start 106.472527 156.468657) (end 106.472527 155.193656) (width 0.2) (layer "F.Cu") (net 30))
 (segment (start 106.472527 155.193656) (end 106.497527 155.168656) (width 0.2) (layer "F.Cu") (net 30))
 (segment (start 106.372527 153.537658) (end 106.372527 153.192657) (width 0.2) (layer "F.Cu") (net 30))
 (segment (start 106.972527 155.193656) (end 106.947527 155.168656) (width 0.2) (layer "F.Cu") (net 1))
 (segment (start 106.947527 155.168656) (end 106.947527 153.662658) (width 0.2) (layer "F.Cu") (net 1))
 (segment (start 106.947527 153.662658) (end 107.072527 153.537658) (width 0.2) (layer "F.Cu") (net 1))
 (segment (start 106.972527 156.468657) (end 106.972527 155.193656) (width 0.2) (layer "F.Cu") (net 1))
 (segment (start 107.072527 153.537658) (end 107.072527 153.192657) (width 0.2) (layer "F.Cu") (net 1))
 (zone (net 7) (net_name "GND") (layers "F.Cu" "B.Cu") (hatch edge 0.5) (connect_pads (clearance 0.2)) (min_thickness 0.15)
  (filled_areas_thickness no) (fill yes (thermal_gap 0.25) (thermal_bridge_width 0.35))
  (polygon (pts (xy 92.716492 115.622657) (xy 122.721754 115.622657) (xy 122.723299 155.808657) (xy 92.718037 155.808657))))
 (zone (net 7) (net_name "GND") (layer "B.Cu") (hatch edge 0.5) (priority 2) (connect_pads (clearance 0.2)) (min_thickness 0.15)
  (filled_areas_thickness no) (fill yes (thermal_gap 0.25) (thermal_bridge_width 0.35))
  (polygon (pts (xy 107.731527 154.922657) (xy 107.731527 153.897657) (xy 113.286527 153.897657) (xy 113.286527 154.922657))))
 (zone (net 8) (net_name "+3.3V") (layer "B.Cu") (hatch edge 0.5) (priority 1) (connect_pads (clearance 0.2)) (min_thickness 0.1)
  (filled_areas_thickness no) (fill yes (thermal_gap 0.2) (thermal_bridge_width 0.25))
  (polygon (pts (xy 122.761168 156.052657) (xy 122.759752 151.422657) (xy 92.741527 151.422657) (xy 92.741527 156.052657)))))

